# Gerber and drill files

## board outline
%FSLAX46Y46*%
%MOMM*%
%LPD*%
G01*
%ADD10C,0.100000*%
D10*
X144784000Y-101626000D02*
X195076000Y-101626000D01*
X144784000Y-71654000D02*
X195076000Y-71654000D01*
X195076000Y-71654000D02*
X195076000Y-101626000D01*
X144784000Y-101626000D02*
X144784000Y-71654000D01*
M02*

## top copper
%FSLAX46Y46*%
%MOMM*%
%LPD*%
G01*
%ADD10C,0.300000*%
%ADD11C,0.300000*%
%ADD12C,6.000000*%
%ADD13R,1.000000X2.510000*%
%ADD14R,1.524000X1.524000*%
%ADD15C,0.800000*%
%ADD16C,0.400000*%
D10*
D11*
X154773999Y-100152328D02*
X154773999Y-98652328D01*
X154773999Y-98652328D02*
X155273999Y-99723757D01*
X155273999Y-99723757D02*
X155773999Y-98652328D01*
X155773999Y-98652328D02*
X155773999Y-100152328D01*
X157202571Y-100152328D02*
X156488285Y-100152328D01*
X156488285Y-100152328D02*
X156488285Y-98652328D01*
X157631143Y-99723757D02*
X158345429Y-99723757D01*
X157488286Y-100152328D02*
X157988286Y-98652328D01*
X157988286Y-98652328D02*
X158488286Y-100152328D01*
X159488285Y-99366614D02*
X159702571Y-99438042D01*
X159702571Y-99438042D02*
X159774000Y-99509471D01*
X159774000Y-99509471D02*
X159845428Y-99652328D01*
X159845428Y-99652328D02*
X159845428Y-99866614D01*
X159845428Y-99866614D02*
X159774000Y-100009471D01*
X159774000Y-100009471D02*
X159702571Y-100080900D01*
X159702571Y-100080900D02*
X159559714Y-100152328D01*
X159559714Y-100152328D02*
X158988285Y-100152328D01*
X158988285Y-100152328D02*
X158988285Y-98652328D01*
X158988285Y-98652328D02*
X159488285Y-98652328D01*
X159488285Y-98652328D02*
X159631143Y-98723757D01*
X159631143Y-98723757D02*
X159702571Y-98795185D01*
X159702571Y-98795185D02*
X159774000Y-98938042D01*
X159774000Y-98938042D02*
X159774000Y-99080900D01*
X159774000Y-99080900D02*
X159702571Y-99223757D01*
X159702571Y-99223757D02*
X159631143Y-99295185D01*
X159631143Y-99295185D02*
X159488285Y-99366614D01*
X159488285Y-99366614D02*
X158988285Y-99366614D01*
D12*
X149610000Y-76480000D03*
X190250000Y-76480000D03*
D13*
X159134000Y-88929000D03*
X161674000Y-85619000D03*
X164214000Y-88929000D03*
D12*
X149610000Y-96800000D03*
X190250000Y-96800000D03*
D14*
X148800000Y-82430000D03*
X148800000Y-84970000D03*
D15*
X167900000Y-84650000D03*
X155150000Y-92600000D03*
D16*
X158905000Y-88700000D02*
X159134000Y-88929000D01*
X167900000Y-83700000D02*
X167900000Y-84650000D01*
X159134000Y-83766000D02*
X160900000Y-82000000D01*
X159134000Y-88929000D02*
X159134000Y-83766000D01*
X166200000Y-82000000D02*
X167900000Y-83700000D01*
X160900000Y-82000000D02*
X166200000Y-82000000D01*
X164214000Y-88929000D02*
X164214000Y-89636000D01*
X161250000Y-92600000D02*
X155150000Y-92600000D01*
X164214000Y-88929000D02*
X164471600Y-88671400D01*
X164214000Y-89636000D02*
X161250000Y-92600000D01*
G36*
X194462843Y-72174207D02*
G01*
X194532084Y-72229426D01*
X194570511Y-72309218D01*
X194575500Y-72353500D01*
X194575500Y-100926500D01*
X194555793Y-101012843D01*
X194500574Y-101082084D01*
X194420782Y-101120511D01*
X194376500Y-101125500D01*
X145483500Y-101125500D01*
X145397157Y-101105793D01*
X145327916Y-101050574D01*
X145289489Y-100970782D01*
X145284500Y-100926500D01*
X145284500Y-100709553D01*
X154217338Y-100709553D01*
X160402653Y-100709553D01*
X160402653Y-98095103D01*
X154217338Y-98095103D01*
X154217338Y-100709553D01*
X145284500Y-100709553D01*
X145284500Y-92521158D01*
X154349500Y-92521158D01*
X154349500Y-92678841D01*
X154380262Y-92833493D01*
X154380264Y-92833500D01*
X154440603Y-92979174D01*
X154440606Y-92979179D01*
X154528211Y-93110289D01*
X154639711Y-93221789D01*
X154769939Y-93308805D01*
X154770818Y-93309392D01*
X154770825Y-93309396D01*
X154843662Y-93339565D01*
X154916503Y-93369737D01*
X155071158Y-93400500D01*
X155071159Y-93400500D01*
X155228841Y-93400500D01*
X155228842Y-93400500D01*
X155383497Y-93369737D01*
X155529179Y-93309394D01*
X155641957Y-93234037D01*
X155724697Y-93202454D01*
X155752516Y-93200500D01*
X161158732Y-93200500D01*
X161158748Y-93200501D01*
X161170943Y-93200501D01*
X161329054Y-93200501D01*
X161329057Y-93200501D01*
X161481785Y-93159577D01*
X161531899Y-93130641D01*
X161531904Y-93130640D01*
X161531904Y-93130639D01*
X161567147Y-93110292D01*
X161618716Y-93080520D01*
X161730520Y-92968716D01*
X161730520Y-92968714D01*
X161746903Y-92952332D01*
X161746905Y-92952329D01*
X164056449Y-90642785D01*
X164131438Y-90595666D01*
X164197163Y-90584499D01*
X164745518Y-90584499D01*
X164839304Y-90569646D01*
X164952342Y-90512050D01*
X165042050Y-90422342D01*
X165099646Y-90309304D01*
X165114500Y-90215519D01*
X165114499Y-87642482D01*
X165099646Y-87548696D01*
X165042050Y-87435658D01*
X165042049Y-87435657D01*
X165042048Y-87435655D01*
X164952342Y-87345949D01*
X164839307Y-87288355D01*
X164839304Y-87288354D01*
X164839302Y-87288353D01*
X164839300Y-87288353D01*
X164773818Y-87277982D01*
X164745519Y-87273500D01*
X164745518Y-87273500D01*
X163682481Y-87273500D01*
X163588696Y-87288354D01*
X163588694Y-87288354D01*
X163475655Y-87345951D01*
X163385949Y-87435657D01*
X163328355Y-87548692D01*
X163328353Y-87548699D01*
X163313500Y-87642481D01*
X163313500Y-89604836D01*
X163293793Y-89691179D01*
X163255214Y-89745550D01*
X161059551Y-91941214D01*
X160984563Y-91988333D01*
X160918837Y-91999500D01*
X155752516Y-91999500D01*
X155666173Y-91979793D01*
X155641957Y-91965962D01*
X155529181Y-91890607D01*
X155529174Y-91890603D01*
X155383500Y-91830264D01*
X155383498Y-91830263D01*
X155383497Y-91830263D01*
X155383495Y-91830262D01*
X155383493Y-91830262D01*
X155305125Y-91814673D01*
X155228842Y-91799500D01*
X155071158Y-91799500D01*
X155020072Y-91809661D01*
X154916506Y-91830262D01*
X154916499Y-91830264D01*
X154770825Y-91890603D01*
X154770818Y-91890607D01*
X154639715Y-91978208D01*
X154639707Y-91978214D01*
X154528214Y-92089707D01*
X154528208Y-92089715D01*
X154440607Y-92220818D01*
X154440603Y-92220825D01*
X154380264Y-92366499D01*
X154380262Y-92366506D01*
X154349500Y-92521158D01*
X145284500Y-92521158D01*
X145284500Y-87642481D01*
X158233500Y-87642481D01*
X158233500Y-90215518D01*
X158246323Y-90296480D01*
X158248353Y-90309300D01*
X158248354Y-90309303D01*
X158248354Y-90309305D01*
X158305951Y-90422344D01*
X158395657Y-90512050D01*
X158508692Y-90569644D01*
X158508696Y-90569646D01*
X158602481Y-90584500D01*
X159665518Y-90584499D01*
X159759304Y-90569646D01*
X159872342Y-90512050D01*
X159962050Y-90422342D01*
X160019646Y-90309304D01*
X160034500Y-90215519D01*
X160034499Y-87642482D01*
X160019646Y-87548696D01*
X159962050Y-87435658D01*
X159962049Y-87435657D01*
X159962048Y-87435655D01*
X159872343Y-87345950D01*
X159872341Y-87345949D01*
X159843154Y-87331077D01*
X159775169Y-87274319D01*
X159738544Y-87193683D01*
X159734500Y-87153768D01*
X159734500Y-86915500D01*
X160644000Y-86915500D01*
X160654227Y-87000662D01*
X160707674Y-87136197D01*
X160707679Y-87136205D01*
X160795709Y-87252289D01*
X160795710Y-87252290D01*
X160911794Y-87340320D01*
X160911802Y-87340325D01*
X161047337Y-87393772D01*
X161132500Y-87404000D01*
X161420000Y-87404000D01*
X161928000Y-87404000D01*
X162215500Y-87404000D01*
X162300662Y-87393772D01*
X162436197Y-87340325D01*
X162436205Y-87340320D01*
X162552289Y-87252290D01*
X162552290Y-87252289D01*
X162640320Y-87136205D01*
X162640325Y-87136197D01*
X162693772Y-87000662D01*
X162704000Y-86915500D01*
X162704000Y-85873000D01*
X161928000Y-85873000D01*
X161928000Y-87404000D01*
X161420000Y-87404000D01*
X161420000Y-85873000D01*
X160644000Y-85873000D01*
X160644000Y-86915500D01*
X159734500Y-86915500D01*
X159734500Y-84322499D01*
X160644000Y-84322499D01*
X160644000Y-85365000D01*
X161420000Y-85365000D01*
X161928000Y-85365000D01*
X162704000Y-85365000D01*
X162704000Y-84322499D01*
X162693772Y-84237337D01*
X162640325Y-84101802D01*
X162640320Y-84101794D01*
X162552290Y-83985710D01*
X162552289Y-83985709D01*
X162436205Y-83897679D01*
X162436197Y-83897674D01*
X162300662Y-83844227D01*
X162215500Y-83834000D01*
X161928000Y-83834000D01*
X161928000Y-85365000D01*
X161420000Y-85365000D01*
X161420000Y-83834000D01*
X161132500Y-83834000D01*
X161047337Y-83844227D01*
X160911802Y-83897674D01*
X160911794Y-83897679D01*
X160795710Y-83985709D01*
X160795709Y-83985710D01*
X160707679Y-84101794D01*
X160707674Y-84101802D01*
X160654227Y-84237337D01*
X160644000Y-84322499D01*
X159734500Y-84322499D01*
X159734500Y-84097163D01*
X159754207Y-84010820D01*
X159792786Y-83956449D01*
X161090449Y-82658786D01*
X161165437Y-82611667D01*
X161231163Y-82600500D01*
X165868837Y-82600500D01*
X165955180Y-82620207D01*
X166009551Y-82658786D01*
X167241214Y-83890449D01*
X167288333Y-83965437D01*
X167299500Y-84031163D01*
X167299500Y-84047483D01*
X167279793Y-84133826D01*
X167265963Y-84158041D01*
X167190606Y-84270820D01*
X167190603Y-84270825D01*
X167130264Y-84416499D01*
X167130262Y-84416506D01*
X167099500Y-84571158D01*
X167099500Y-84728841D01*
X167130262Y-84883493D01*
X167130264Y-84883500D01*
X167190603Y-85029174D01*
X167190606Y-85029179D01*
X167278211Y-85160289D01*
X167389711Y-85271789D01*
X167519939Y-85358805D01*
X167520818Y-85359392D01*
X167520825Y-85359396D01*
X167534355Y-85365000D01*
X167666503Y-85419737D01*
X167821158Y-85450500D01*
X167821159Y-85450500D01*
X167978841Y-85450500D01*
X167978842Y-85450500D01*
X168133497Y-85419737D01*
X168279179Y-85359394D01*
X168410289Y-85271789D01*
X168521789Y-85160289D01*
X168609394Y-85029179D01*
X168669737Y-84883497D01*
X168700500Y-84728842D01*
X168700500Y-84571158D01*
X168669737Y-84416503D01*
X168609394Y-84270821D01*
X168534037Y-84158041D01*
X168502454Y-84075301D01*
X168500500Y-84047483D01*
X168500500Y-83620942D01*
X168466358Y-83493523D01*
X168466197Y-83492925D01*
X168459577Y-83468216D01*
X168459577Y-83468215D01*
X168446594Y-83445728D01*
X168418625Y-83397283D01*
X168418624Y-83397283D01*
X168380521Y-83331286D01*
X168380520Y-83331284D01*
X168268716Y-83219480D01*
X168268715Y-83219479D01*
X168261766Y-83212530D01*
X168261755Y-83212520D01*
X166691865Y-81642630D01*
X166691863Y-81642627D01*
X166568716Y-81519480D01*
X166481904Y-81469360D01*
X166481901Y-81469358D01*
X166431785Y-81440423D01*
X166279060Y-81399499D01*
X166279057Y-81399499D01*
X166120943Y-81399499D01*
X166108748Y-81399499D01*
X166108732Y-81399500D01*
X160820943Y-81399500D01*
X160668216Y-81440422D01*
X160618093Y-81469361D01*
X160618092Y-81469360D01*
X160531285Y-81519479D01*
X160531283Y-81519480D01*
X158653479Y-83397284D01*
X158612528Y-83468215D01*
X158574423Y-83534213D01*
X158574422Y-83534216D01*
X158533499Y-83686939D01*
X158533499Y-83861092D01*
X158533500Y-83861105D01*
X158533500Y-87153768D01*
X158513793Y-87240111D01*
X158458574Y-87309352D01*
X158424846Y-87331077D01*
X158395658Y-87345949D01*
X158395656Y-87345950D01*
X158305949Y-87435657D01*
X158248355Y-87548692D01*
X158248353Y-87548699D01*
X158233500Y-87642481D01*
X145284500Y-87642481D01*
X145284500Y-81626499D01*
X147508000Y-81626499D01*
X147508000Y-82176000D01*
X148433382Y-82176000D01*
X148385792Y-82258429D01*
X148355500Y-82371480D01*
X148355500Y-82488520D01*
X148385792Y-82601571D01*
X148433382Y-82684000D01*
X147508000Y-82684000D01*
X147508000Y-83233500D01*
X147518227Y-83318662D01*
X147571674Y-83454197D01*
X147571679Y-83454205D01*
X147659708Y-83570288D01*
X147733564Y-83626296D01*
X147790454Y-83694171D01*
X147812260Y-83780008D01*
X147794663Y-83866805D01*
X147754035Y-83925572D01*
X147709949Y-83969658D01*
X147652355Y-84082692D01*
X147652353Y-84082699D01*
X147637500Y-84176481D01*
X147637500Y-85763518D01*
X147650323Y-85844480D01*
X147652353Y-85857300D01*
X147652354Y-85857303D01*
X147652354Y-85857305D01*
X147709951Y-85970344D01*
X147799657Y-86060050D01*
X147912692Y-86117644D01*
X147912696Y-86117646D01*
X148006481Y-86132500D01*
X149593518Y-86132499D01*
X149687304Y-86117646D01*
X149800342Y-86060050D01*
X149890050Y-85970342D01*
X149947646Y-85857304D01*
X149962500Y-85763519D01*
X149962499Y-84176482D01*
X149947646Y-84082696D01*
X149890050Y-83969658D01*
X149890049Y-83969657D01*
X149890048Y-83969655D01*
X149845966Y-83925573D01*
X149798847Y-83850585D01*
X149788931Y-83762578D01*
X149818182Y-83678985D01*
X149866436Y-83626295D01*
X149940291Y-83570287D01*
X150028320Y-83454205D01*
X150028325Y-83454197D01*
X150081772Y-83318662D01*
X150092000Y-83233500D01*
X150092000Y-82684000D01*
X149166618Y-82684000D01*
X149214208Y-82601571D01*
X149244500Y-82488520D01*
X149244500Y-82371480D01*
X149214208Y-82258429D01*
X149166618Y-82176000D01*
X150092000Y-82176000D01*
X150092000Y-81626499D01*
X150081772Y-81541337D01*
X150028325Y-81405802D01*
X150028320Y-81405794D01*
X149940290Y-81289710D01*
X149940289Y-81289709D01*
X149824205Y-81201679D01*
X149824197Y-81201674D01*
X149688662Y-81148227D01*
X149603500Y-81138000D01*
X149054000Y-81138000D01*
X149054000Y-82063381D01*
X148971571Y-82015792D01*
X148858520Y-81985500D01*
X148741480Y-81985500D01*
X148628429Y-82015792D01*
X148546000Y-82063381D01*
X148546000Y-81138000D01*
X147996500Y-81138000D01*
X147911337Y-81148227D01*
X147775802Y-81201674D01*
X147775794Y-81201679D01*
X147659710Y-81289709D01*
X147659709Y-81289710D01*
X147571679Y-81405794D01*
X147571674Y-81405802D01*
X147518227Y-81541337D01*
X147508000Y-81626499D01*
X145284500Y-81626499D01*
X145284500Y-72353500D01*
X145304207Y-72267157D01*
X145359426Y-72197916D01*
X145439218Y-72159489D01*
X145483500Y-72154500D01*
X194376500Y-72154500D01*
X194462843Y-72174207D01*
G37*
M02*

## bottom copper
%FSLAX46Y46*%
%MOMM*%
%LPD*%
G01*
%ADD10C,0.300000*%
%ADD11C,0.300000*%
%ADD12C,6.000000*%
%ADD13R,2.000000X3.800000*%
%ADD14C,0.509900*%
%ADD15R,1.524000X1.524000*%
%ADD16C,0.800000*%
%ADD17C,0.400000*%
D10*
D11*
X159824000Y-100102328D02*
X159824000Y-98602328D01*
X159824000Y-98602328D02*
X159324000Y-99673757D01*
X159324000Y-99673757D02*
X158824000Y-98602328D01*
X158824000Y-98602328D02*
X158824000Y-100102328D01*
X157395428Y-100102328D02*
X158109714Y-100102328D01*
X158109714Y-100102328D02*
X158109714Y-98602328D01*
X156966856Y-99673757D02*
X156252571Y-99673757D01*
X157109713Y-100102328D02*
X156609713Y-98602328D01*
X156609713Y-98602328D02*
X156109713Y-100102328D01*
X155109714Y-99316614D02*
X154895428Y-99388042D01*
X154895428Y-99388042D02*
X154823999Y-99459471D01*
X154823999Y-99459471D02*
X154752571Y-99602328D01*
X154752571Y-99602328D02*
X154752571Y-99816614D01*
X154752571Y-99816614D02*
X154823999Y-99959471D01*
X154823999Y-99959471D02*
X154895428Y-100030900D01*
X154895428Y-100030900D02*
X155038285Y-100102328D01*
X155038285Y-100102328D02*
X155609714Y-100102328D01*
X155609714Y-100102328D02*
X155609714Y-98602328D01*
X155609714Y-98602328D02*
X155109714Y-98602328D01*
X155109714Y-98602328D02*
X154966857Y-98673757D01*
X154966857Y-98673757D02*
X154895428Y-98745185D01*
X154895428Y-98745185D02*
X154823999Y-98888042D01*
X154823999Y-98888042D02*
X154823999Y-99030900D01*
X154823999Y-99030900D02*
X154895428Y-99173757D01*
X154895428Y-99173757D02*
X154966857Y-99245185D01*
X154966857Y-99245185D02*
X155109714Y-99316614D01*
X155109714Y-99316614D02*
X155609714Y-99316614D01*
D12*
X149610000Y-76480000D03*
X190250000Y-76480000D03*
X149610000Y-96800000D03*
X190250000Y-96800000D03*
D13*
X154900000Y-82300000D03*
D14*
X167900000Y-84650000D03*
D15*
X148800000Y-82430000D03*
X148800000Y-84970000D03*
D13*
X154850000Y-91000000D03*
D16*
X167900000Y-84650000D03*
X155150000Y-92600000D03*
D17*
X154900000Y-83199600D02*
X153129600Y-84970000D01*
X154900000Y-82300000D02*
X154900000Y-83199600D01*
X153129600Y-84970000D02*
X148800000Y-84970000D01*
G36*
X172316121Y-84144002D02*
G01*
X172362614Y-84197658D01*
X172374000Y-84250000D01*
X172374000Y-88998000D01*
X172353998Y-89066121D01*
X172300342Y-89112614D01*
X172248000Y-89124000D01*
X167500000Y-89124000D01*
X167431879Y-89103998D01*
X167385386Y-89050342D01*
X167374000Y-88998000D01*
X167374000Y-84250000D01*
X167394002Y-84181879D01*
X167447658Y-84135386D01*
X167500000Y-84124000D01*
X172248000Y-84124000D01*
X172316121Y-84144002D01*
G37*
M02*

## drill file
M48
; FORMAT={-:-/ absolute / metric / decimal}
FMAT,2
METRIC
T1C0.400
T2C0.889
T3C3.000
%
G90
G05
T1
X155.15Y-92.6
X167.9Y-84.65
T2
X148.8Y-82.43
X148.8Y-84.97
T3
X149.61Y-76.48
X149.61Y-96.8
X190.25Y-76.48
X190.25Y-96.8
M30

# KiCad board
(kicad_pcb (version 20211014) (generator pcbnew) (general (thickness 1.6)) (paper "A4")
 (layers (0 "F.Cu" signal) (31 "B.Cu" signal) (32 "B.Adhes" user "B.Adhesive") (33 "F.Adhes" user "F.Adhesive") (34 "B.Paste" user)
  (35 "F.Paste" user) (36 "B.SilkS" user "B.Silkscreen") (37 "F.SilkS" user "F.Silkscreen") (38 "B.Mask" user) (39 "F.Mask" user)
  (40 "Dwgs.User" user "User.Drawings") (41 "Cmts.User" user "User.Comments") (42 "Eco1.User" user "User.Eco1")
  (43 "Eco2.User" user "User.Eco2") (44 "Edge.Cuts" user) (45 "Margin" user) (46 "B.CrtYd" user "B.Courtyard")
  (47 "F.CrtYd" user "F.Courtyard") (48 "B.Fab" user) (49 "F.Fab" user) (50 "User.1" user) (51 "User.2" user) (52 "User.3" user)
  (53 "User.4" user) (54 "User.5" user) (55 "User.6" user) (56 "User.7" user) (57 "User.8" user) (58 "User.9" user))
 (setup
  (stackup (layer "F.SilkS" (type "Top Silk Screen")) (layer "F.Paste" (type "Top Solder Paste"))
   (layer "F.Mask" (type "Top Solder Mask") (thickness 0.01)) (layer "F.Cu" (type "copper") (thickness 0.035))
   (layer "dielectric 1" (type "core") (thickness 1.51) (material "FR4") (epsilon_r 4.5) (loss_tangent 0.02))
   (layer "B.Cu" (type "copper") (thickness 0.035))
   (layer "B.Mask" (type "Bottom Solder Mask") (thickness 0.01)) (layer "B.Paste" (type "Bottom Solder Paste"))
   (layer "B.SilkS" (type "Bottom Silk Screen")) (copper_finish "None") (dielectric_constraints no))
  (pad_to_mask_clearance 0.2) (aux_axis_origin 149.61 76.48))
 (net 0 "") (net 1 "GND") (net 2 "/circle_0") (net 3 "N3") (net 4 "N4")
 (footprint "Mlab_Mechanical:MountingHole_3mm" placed (layer "F.Cu") (at 149.61 76.48)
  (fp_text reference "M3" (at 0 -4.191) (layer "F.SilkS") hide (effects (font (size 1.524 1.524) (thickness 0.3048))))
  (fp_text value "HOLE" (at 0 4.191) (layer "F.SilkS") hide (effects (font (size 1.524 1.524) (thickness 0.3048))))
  (pad "1" thru_hole circle (at 0 0) (size 6 6) (drill 3) (layers *.Cu *.Mask) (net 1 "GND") (clearance 1) (zone_connect 2)))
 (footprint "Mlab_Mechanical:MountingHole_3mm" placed (layer "F.Cu") (at 190.25 76.48)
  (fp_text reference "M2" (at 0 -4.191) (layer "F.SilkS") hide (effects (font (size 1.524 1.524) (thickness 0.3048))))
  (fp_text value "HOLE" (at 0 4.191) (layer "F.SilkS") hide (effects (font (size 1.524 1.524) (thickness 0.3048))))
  (pad "1" thru_hole circle (at 0 0) (size 6 6) (drill 3) (layers *.Cu *.Mask) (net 1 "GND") (clearance 1) (zone_connect 2)))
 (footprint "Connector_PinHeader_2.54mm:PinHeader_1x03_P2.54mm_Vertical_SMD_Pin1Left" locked (layer "F.Cu") (at 161.674 87.274 90)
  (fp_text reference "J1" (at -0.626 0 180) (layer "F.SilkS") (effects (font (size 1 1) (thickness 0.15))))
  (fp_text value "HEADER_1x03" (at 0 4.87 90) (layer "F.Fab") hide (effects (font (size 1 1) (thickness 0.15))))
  (pad "1" smd rect locked (at -1.655 -2.54 90) (size 2.51 1) (layers "F.Cu" "F.Paste" "F.Mask") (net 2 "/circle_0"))
  (pad "2" smd rect locked (at 1.655 0 90) (size 2.51 1) (layers "F.Cu" "F.Paste" "F.Mask") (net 1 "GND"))
  (pad "3" smd rect locked (at -1.655 2.54 90) (size 2.51 1) (layers "F.Cu" "F.Paste" "F.Mask") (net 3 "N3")))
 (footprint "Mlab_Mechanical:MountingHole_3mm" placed (layer "F.Cu") (at 149.61 96.8)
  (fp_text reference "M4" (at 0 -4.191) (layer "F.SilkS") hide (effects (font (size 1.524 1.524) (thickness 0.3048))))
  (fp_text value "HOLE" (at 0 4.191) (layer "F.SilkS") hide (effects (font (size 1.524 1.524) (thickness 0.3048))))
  (pad "1" thru_hole circle (at 0 0) (size 6 6) (drill 3) (layers *.Cu *.Mask) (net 1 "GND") (clearance 1) (zone_connect 2)))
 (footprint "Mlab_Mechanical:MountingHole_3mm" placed (layer "F.Cu") (at 190.25 96.8)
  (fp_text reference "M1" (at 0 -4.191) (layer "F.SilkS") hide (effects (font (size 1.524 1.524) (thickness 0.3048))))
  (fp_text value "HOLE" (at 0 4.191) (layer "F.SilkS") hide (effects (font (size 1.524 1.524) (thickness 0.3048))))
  (pad "1" thru_hole circle (at 0 0) (size 6 6) (drill 3) (layers *.Cu *.Mask) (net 1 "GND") (clearance 1) (zone_connect 2)))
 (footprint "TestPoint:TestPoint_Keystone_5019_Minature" (layer "B.Cu") (at 154.9 82.3 -90) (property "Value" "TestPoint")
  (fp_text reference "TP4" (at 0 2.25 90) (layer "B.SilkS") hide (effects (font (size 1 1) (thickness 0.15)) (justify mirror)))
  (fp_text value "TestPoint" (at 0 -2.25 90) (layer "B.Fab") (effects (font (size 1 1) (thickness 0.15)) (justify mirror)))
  (pad "1" smd rect (at 0 0 270) (size 3.8 2) (layers "B.Cu" "B.Paste" "B.Mask") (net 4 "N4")))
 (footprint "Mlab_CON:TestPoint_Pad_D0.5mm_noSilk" (layer "B.Cu") (at 167.9 84.65 180) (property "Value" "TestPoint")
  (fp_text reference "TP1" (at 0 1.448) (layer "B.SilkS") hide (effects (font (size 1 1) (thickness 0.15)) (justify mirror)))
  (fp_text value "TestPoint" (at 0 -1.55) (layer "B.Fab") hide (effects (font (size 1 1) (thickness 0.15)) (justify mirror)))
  (pad "1" smd circle (at 0 0 180) (size 0.5099 0.5099) (layers "B.Cu" "B.Mask") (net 2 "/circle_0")))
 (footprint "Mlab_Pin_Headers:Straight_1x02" (layer "B.Cu") (at 148.8 83.7 180)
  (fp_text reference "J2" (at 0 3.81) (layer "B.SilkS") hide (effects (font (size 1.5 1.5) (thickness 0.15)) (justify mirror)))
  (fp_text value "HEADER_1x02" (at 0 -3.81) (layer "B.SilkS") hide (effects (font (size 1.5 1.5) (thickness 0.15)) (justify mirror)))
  (pad "1" thru_hole rect (at 0 1.27 180) (size 1.524 1.524) (drill 0.889) (layers *.Cu *.Mask "B.SilkS") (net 1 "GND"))
  (pad "2" thru_hole rect (at 0 -1.27 180) (size 1.524 1.524) (drill 0.889) (layers *.Cu *.Mask "B.SilkS") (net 4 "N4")))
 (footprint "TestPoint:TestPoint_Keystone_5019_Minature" (layer "B.Cu") (at 154.85 91 90) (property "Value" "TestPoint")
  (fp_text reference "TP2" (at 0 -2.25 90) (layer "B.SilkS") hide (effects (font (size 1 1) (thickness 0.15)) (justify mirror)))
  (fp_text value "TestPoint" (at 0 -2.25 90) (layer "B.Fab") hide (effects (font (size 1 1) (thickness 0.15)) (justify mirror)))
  (pad "1" smd rect (at 0 0 90) (size 3.8 2) (layers "B.Cu" "B.Paste" "B.Mask") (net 3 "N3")))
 (gr_line (start 144.784 101.626) (end 195.076 101.626) (layer "Edge.Cuts") (width 0.1))
 (gr_line (start 144.784 71.654) (end 195.076 71.654) (layer "Edge.Cuts") (width 0.1))
 (gr_line (start 195.076 71.654) (end 195.076 101.626) (layer "Edge.Cuts") (width 0.1))
 (gr_line (start 144.784 101.626) (end 144.784 71.654) (layer "Edge.Cuts") (width 0.1))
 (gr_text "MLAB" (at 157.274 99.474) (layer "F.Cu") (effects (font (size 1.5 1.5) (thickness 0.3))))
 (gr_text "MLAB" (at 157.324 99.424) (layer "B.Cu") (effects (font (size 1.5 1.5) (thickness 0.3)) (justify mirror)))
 (segment (start 158.905 88.7) (end 159.134 88.929) (width 0.4) (layer "F.Cu") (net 2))
 (segment (start 167.9 83.7) (end 167.9 84.65) (width 0.4) (layer "F.Cu") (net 2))
 (segment (start 159.134 83.766) (end 160.9 82) (width 0.4) (layer "F.Cu") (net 2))
 (segment (start 159.134 88.929) (end 159.134 83.766) (width 0.4) (layer "F.Cu") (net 2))
 (segment (start 166.2 82) (end 167.9 83.7) (width 0.4) (layer "F.Cu") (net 2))
 (segment (start 160.9 82) (end 166.2 82) (width 0.4) (layer "F.Cu") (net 2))
 (via (at 167.9 84.65) (size 0.8) (drill 0.4) (layers "F.Cu" "B.Cu") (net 2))
 (segment (start 164.214 88.929) (end 164.214 89.636) (width 0.4) (layer "F.Cu") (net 3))
 (segment (start 161.25 92.6) (end 155.15 92.6) (width 0.4) (layer "F.Cu") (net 3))
 (segment (start 164.214 88.929) (end 164.4716 88.6714) (width 0.4) (layer "F.Cu") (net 3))
 (segment (start 164.214 89.636) (end 161.25 92.6) (width 0.4) (layer "F.Cu") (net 3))
 (via (at 155.15 92.6) (size 0.8) (drill 0.4) (layers "F.Cu" "B.Cu") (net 3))
 (segment (start 154.9 83.1996) (end 153.1296 84.97) (width 0.4) (layer "B.Cu") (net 4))
 (segment (start 154.9 82.3) (end 154.9 83.1996) (width 0.4) (layer "B.Cu") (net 4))
 (segment (start 153.1296 84.97) (end 148.8 84.97) (width 0.4) (layer "B.Cu") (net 4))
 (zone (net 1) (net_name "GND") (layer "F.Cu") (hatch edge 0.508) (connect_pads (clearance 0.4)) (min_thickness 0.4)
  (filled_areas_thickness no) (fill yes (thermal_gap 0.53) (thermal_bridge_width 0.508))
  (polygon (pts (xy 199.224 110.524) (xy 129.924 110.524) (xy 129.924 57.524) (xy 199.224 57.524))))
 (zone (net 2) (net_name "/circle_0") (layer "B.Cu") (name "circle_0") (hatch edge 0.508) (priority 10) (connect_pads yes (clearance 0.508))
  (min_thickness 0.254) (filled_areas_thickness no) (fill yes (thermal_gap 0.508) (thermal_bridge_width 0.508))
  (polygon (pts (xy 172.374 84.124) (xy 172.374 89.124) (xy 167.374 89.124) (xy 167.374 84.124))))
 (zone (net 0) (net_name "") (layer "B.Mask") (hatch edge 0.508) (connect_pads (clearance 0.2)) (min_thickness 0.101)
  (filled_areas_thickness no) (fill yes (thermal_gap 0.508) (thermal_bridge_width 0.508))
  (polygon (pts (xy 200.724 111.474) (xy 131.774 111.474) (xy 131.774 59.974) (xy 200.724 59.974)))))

